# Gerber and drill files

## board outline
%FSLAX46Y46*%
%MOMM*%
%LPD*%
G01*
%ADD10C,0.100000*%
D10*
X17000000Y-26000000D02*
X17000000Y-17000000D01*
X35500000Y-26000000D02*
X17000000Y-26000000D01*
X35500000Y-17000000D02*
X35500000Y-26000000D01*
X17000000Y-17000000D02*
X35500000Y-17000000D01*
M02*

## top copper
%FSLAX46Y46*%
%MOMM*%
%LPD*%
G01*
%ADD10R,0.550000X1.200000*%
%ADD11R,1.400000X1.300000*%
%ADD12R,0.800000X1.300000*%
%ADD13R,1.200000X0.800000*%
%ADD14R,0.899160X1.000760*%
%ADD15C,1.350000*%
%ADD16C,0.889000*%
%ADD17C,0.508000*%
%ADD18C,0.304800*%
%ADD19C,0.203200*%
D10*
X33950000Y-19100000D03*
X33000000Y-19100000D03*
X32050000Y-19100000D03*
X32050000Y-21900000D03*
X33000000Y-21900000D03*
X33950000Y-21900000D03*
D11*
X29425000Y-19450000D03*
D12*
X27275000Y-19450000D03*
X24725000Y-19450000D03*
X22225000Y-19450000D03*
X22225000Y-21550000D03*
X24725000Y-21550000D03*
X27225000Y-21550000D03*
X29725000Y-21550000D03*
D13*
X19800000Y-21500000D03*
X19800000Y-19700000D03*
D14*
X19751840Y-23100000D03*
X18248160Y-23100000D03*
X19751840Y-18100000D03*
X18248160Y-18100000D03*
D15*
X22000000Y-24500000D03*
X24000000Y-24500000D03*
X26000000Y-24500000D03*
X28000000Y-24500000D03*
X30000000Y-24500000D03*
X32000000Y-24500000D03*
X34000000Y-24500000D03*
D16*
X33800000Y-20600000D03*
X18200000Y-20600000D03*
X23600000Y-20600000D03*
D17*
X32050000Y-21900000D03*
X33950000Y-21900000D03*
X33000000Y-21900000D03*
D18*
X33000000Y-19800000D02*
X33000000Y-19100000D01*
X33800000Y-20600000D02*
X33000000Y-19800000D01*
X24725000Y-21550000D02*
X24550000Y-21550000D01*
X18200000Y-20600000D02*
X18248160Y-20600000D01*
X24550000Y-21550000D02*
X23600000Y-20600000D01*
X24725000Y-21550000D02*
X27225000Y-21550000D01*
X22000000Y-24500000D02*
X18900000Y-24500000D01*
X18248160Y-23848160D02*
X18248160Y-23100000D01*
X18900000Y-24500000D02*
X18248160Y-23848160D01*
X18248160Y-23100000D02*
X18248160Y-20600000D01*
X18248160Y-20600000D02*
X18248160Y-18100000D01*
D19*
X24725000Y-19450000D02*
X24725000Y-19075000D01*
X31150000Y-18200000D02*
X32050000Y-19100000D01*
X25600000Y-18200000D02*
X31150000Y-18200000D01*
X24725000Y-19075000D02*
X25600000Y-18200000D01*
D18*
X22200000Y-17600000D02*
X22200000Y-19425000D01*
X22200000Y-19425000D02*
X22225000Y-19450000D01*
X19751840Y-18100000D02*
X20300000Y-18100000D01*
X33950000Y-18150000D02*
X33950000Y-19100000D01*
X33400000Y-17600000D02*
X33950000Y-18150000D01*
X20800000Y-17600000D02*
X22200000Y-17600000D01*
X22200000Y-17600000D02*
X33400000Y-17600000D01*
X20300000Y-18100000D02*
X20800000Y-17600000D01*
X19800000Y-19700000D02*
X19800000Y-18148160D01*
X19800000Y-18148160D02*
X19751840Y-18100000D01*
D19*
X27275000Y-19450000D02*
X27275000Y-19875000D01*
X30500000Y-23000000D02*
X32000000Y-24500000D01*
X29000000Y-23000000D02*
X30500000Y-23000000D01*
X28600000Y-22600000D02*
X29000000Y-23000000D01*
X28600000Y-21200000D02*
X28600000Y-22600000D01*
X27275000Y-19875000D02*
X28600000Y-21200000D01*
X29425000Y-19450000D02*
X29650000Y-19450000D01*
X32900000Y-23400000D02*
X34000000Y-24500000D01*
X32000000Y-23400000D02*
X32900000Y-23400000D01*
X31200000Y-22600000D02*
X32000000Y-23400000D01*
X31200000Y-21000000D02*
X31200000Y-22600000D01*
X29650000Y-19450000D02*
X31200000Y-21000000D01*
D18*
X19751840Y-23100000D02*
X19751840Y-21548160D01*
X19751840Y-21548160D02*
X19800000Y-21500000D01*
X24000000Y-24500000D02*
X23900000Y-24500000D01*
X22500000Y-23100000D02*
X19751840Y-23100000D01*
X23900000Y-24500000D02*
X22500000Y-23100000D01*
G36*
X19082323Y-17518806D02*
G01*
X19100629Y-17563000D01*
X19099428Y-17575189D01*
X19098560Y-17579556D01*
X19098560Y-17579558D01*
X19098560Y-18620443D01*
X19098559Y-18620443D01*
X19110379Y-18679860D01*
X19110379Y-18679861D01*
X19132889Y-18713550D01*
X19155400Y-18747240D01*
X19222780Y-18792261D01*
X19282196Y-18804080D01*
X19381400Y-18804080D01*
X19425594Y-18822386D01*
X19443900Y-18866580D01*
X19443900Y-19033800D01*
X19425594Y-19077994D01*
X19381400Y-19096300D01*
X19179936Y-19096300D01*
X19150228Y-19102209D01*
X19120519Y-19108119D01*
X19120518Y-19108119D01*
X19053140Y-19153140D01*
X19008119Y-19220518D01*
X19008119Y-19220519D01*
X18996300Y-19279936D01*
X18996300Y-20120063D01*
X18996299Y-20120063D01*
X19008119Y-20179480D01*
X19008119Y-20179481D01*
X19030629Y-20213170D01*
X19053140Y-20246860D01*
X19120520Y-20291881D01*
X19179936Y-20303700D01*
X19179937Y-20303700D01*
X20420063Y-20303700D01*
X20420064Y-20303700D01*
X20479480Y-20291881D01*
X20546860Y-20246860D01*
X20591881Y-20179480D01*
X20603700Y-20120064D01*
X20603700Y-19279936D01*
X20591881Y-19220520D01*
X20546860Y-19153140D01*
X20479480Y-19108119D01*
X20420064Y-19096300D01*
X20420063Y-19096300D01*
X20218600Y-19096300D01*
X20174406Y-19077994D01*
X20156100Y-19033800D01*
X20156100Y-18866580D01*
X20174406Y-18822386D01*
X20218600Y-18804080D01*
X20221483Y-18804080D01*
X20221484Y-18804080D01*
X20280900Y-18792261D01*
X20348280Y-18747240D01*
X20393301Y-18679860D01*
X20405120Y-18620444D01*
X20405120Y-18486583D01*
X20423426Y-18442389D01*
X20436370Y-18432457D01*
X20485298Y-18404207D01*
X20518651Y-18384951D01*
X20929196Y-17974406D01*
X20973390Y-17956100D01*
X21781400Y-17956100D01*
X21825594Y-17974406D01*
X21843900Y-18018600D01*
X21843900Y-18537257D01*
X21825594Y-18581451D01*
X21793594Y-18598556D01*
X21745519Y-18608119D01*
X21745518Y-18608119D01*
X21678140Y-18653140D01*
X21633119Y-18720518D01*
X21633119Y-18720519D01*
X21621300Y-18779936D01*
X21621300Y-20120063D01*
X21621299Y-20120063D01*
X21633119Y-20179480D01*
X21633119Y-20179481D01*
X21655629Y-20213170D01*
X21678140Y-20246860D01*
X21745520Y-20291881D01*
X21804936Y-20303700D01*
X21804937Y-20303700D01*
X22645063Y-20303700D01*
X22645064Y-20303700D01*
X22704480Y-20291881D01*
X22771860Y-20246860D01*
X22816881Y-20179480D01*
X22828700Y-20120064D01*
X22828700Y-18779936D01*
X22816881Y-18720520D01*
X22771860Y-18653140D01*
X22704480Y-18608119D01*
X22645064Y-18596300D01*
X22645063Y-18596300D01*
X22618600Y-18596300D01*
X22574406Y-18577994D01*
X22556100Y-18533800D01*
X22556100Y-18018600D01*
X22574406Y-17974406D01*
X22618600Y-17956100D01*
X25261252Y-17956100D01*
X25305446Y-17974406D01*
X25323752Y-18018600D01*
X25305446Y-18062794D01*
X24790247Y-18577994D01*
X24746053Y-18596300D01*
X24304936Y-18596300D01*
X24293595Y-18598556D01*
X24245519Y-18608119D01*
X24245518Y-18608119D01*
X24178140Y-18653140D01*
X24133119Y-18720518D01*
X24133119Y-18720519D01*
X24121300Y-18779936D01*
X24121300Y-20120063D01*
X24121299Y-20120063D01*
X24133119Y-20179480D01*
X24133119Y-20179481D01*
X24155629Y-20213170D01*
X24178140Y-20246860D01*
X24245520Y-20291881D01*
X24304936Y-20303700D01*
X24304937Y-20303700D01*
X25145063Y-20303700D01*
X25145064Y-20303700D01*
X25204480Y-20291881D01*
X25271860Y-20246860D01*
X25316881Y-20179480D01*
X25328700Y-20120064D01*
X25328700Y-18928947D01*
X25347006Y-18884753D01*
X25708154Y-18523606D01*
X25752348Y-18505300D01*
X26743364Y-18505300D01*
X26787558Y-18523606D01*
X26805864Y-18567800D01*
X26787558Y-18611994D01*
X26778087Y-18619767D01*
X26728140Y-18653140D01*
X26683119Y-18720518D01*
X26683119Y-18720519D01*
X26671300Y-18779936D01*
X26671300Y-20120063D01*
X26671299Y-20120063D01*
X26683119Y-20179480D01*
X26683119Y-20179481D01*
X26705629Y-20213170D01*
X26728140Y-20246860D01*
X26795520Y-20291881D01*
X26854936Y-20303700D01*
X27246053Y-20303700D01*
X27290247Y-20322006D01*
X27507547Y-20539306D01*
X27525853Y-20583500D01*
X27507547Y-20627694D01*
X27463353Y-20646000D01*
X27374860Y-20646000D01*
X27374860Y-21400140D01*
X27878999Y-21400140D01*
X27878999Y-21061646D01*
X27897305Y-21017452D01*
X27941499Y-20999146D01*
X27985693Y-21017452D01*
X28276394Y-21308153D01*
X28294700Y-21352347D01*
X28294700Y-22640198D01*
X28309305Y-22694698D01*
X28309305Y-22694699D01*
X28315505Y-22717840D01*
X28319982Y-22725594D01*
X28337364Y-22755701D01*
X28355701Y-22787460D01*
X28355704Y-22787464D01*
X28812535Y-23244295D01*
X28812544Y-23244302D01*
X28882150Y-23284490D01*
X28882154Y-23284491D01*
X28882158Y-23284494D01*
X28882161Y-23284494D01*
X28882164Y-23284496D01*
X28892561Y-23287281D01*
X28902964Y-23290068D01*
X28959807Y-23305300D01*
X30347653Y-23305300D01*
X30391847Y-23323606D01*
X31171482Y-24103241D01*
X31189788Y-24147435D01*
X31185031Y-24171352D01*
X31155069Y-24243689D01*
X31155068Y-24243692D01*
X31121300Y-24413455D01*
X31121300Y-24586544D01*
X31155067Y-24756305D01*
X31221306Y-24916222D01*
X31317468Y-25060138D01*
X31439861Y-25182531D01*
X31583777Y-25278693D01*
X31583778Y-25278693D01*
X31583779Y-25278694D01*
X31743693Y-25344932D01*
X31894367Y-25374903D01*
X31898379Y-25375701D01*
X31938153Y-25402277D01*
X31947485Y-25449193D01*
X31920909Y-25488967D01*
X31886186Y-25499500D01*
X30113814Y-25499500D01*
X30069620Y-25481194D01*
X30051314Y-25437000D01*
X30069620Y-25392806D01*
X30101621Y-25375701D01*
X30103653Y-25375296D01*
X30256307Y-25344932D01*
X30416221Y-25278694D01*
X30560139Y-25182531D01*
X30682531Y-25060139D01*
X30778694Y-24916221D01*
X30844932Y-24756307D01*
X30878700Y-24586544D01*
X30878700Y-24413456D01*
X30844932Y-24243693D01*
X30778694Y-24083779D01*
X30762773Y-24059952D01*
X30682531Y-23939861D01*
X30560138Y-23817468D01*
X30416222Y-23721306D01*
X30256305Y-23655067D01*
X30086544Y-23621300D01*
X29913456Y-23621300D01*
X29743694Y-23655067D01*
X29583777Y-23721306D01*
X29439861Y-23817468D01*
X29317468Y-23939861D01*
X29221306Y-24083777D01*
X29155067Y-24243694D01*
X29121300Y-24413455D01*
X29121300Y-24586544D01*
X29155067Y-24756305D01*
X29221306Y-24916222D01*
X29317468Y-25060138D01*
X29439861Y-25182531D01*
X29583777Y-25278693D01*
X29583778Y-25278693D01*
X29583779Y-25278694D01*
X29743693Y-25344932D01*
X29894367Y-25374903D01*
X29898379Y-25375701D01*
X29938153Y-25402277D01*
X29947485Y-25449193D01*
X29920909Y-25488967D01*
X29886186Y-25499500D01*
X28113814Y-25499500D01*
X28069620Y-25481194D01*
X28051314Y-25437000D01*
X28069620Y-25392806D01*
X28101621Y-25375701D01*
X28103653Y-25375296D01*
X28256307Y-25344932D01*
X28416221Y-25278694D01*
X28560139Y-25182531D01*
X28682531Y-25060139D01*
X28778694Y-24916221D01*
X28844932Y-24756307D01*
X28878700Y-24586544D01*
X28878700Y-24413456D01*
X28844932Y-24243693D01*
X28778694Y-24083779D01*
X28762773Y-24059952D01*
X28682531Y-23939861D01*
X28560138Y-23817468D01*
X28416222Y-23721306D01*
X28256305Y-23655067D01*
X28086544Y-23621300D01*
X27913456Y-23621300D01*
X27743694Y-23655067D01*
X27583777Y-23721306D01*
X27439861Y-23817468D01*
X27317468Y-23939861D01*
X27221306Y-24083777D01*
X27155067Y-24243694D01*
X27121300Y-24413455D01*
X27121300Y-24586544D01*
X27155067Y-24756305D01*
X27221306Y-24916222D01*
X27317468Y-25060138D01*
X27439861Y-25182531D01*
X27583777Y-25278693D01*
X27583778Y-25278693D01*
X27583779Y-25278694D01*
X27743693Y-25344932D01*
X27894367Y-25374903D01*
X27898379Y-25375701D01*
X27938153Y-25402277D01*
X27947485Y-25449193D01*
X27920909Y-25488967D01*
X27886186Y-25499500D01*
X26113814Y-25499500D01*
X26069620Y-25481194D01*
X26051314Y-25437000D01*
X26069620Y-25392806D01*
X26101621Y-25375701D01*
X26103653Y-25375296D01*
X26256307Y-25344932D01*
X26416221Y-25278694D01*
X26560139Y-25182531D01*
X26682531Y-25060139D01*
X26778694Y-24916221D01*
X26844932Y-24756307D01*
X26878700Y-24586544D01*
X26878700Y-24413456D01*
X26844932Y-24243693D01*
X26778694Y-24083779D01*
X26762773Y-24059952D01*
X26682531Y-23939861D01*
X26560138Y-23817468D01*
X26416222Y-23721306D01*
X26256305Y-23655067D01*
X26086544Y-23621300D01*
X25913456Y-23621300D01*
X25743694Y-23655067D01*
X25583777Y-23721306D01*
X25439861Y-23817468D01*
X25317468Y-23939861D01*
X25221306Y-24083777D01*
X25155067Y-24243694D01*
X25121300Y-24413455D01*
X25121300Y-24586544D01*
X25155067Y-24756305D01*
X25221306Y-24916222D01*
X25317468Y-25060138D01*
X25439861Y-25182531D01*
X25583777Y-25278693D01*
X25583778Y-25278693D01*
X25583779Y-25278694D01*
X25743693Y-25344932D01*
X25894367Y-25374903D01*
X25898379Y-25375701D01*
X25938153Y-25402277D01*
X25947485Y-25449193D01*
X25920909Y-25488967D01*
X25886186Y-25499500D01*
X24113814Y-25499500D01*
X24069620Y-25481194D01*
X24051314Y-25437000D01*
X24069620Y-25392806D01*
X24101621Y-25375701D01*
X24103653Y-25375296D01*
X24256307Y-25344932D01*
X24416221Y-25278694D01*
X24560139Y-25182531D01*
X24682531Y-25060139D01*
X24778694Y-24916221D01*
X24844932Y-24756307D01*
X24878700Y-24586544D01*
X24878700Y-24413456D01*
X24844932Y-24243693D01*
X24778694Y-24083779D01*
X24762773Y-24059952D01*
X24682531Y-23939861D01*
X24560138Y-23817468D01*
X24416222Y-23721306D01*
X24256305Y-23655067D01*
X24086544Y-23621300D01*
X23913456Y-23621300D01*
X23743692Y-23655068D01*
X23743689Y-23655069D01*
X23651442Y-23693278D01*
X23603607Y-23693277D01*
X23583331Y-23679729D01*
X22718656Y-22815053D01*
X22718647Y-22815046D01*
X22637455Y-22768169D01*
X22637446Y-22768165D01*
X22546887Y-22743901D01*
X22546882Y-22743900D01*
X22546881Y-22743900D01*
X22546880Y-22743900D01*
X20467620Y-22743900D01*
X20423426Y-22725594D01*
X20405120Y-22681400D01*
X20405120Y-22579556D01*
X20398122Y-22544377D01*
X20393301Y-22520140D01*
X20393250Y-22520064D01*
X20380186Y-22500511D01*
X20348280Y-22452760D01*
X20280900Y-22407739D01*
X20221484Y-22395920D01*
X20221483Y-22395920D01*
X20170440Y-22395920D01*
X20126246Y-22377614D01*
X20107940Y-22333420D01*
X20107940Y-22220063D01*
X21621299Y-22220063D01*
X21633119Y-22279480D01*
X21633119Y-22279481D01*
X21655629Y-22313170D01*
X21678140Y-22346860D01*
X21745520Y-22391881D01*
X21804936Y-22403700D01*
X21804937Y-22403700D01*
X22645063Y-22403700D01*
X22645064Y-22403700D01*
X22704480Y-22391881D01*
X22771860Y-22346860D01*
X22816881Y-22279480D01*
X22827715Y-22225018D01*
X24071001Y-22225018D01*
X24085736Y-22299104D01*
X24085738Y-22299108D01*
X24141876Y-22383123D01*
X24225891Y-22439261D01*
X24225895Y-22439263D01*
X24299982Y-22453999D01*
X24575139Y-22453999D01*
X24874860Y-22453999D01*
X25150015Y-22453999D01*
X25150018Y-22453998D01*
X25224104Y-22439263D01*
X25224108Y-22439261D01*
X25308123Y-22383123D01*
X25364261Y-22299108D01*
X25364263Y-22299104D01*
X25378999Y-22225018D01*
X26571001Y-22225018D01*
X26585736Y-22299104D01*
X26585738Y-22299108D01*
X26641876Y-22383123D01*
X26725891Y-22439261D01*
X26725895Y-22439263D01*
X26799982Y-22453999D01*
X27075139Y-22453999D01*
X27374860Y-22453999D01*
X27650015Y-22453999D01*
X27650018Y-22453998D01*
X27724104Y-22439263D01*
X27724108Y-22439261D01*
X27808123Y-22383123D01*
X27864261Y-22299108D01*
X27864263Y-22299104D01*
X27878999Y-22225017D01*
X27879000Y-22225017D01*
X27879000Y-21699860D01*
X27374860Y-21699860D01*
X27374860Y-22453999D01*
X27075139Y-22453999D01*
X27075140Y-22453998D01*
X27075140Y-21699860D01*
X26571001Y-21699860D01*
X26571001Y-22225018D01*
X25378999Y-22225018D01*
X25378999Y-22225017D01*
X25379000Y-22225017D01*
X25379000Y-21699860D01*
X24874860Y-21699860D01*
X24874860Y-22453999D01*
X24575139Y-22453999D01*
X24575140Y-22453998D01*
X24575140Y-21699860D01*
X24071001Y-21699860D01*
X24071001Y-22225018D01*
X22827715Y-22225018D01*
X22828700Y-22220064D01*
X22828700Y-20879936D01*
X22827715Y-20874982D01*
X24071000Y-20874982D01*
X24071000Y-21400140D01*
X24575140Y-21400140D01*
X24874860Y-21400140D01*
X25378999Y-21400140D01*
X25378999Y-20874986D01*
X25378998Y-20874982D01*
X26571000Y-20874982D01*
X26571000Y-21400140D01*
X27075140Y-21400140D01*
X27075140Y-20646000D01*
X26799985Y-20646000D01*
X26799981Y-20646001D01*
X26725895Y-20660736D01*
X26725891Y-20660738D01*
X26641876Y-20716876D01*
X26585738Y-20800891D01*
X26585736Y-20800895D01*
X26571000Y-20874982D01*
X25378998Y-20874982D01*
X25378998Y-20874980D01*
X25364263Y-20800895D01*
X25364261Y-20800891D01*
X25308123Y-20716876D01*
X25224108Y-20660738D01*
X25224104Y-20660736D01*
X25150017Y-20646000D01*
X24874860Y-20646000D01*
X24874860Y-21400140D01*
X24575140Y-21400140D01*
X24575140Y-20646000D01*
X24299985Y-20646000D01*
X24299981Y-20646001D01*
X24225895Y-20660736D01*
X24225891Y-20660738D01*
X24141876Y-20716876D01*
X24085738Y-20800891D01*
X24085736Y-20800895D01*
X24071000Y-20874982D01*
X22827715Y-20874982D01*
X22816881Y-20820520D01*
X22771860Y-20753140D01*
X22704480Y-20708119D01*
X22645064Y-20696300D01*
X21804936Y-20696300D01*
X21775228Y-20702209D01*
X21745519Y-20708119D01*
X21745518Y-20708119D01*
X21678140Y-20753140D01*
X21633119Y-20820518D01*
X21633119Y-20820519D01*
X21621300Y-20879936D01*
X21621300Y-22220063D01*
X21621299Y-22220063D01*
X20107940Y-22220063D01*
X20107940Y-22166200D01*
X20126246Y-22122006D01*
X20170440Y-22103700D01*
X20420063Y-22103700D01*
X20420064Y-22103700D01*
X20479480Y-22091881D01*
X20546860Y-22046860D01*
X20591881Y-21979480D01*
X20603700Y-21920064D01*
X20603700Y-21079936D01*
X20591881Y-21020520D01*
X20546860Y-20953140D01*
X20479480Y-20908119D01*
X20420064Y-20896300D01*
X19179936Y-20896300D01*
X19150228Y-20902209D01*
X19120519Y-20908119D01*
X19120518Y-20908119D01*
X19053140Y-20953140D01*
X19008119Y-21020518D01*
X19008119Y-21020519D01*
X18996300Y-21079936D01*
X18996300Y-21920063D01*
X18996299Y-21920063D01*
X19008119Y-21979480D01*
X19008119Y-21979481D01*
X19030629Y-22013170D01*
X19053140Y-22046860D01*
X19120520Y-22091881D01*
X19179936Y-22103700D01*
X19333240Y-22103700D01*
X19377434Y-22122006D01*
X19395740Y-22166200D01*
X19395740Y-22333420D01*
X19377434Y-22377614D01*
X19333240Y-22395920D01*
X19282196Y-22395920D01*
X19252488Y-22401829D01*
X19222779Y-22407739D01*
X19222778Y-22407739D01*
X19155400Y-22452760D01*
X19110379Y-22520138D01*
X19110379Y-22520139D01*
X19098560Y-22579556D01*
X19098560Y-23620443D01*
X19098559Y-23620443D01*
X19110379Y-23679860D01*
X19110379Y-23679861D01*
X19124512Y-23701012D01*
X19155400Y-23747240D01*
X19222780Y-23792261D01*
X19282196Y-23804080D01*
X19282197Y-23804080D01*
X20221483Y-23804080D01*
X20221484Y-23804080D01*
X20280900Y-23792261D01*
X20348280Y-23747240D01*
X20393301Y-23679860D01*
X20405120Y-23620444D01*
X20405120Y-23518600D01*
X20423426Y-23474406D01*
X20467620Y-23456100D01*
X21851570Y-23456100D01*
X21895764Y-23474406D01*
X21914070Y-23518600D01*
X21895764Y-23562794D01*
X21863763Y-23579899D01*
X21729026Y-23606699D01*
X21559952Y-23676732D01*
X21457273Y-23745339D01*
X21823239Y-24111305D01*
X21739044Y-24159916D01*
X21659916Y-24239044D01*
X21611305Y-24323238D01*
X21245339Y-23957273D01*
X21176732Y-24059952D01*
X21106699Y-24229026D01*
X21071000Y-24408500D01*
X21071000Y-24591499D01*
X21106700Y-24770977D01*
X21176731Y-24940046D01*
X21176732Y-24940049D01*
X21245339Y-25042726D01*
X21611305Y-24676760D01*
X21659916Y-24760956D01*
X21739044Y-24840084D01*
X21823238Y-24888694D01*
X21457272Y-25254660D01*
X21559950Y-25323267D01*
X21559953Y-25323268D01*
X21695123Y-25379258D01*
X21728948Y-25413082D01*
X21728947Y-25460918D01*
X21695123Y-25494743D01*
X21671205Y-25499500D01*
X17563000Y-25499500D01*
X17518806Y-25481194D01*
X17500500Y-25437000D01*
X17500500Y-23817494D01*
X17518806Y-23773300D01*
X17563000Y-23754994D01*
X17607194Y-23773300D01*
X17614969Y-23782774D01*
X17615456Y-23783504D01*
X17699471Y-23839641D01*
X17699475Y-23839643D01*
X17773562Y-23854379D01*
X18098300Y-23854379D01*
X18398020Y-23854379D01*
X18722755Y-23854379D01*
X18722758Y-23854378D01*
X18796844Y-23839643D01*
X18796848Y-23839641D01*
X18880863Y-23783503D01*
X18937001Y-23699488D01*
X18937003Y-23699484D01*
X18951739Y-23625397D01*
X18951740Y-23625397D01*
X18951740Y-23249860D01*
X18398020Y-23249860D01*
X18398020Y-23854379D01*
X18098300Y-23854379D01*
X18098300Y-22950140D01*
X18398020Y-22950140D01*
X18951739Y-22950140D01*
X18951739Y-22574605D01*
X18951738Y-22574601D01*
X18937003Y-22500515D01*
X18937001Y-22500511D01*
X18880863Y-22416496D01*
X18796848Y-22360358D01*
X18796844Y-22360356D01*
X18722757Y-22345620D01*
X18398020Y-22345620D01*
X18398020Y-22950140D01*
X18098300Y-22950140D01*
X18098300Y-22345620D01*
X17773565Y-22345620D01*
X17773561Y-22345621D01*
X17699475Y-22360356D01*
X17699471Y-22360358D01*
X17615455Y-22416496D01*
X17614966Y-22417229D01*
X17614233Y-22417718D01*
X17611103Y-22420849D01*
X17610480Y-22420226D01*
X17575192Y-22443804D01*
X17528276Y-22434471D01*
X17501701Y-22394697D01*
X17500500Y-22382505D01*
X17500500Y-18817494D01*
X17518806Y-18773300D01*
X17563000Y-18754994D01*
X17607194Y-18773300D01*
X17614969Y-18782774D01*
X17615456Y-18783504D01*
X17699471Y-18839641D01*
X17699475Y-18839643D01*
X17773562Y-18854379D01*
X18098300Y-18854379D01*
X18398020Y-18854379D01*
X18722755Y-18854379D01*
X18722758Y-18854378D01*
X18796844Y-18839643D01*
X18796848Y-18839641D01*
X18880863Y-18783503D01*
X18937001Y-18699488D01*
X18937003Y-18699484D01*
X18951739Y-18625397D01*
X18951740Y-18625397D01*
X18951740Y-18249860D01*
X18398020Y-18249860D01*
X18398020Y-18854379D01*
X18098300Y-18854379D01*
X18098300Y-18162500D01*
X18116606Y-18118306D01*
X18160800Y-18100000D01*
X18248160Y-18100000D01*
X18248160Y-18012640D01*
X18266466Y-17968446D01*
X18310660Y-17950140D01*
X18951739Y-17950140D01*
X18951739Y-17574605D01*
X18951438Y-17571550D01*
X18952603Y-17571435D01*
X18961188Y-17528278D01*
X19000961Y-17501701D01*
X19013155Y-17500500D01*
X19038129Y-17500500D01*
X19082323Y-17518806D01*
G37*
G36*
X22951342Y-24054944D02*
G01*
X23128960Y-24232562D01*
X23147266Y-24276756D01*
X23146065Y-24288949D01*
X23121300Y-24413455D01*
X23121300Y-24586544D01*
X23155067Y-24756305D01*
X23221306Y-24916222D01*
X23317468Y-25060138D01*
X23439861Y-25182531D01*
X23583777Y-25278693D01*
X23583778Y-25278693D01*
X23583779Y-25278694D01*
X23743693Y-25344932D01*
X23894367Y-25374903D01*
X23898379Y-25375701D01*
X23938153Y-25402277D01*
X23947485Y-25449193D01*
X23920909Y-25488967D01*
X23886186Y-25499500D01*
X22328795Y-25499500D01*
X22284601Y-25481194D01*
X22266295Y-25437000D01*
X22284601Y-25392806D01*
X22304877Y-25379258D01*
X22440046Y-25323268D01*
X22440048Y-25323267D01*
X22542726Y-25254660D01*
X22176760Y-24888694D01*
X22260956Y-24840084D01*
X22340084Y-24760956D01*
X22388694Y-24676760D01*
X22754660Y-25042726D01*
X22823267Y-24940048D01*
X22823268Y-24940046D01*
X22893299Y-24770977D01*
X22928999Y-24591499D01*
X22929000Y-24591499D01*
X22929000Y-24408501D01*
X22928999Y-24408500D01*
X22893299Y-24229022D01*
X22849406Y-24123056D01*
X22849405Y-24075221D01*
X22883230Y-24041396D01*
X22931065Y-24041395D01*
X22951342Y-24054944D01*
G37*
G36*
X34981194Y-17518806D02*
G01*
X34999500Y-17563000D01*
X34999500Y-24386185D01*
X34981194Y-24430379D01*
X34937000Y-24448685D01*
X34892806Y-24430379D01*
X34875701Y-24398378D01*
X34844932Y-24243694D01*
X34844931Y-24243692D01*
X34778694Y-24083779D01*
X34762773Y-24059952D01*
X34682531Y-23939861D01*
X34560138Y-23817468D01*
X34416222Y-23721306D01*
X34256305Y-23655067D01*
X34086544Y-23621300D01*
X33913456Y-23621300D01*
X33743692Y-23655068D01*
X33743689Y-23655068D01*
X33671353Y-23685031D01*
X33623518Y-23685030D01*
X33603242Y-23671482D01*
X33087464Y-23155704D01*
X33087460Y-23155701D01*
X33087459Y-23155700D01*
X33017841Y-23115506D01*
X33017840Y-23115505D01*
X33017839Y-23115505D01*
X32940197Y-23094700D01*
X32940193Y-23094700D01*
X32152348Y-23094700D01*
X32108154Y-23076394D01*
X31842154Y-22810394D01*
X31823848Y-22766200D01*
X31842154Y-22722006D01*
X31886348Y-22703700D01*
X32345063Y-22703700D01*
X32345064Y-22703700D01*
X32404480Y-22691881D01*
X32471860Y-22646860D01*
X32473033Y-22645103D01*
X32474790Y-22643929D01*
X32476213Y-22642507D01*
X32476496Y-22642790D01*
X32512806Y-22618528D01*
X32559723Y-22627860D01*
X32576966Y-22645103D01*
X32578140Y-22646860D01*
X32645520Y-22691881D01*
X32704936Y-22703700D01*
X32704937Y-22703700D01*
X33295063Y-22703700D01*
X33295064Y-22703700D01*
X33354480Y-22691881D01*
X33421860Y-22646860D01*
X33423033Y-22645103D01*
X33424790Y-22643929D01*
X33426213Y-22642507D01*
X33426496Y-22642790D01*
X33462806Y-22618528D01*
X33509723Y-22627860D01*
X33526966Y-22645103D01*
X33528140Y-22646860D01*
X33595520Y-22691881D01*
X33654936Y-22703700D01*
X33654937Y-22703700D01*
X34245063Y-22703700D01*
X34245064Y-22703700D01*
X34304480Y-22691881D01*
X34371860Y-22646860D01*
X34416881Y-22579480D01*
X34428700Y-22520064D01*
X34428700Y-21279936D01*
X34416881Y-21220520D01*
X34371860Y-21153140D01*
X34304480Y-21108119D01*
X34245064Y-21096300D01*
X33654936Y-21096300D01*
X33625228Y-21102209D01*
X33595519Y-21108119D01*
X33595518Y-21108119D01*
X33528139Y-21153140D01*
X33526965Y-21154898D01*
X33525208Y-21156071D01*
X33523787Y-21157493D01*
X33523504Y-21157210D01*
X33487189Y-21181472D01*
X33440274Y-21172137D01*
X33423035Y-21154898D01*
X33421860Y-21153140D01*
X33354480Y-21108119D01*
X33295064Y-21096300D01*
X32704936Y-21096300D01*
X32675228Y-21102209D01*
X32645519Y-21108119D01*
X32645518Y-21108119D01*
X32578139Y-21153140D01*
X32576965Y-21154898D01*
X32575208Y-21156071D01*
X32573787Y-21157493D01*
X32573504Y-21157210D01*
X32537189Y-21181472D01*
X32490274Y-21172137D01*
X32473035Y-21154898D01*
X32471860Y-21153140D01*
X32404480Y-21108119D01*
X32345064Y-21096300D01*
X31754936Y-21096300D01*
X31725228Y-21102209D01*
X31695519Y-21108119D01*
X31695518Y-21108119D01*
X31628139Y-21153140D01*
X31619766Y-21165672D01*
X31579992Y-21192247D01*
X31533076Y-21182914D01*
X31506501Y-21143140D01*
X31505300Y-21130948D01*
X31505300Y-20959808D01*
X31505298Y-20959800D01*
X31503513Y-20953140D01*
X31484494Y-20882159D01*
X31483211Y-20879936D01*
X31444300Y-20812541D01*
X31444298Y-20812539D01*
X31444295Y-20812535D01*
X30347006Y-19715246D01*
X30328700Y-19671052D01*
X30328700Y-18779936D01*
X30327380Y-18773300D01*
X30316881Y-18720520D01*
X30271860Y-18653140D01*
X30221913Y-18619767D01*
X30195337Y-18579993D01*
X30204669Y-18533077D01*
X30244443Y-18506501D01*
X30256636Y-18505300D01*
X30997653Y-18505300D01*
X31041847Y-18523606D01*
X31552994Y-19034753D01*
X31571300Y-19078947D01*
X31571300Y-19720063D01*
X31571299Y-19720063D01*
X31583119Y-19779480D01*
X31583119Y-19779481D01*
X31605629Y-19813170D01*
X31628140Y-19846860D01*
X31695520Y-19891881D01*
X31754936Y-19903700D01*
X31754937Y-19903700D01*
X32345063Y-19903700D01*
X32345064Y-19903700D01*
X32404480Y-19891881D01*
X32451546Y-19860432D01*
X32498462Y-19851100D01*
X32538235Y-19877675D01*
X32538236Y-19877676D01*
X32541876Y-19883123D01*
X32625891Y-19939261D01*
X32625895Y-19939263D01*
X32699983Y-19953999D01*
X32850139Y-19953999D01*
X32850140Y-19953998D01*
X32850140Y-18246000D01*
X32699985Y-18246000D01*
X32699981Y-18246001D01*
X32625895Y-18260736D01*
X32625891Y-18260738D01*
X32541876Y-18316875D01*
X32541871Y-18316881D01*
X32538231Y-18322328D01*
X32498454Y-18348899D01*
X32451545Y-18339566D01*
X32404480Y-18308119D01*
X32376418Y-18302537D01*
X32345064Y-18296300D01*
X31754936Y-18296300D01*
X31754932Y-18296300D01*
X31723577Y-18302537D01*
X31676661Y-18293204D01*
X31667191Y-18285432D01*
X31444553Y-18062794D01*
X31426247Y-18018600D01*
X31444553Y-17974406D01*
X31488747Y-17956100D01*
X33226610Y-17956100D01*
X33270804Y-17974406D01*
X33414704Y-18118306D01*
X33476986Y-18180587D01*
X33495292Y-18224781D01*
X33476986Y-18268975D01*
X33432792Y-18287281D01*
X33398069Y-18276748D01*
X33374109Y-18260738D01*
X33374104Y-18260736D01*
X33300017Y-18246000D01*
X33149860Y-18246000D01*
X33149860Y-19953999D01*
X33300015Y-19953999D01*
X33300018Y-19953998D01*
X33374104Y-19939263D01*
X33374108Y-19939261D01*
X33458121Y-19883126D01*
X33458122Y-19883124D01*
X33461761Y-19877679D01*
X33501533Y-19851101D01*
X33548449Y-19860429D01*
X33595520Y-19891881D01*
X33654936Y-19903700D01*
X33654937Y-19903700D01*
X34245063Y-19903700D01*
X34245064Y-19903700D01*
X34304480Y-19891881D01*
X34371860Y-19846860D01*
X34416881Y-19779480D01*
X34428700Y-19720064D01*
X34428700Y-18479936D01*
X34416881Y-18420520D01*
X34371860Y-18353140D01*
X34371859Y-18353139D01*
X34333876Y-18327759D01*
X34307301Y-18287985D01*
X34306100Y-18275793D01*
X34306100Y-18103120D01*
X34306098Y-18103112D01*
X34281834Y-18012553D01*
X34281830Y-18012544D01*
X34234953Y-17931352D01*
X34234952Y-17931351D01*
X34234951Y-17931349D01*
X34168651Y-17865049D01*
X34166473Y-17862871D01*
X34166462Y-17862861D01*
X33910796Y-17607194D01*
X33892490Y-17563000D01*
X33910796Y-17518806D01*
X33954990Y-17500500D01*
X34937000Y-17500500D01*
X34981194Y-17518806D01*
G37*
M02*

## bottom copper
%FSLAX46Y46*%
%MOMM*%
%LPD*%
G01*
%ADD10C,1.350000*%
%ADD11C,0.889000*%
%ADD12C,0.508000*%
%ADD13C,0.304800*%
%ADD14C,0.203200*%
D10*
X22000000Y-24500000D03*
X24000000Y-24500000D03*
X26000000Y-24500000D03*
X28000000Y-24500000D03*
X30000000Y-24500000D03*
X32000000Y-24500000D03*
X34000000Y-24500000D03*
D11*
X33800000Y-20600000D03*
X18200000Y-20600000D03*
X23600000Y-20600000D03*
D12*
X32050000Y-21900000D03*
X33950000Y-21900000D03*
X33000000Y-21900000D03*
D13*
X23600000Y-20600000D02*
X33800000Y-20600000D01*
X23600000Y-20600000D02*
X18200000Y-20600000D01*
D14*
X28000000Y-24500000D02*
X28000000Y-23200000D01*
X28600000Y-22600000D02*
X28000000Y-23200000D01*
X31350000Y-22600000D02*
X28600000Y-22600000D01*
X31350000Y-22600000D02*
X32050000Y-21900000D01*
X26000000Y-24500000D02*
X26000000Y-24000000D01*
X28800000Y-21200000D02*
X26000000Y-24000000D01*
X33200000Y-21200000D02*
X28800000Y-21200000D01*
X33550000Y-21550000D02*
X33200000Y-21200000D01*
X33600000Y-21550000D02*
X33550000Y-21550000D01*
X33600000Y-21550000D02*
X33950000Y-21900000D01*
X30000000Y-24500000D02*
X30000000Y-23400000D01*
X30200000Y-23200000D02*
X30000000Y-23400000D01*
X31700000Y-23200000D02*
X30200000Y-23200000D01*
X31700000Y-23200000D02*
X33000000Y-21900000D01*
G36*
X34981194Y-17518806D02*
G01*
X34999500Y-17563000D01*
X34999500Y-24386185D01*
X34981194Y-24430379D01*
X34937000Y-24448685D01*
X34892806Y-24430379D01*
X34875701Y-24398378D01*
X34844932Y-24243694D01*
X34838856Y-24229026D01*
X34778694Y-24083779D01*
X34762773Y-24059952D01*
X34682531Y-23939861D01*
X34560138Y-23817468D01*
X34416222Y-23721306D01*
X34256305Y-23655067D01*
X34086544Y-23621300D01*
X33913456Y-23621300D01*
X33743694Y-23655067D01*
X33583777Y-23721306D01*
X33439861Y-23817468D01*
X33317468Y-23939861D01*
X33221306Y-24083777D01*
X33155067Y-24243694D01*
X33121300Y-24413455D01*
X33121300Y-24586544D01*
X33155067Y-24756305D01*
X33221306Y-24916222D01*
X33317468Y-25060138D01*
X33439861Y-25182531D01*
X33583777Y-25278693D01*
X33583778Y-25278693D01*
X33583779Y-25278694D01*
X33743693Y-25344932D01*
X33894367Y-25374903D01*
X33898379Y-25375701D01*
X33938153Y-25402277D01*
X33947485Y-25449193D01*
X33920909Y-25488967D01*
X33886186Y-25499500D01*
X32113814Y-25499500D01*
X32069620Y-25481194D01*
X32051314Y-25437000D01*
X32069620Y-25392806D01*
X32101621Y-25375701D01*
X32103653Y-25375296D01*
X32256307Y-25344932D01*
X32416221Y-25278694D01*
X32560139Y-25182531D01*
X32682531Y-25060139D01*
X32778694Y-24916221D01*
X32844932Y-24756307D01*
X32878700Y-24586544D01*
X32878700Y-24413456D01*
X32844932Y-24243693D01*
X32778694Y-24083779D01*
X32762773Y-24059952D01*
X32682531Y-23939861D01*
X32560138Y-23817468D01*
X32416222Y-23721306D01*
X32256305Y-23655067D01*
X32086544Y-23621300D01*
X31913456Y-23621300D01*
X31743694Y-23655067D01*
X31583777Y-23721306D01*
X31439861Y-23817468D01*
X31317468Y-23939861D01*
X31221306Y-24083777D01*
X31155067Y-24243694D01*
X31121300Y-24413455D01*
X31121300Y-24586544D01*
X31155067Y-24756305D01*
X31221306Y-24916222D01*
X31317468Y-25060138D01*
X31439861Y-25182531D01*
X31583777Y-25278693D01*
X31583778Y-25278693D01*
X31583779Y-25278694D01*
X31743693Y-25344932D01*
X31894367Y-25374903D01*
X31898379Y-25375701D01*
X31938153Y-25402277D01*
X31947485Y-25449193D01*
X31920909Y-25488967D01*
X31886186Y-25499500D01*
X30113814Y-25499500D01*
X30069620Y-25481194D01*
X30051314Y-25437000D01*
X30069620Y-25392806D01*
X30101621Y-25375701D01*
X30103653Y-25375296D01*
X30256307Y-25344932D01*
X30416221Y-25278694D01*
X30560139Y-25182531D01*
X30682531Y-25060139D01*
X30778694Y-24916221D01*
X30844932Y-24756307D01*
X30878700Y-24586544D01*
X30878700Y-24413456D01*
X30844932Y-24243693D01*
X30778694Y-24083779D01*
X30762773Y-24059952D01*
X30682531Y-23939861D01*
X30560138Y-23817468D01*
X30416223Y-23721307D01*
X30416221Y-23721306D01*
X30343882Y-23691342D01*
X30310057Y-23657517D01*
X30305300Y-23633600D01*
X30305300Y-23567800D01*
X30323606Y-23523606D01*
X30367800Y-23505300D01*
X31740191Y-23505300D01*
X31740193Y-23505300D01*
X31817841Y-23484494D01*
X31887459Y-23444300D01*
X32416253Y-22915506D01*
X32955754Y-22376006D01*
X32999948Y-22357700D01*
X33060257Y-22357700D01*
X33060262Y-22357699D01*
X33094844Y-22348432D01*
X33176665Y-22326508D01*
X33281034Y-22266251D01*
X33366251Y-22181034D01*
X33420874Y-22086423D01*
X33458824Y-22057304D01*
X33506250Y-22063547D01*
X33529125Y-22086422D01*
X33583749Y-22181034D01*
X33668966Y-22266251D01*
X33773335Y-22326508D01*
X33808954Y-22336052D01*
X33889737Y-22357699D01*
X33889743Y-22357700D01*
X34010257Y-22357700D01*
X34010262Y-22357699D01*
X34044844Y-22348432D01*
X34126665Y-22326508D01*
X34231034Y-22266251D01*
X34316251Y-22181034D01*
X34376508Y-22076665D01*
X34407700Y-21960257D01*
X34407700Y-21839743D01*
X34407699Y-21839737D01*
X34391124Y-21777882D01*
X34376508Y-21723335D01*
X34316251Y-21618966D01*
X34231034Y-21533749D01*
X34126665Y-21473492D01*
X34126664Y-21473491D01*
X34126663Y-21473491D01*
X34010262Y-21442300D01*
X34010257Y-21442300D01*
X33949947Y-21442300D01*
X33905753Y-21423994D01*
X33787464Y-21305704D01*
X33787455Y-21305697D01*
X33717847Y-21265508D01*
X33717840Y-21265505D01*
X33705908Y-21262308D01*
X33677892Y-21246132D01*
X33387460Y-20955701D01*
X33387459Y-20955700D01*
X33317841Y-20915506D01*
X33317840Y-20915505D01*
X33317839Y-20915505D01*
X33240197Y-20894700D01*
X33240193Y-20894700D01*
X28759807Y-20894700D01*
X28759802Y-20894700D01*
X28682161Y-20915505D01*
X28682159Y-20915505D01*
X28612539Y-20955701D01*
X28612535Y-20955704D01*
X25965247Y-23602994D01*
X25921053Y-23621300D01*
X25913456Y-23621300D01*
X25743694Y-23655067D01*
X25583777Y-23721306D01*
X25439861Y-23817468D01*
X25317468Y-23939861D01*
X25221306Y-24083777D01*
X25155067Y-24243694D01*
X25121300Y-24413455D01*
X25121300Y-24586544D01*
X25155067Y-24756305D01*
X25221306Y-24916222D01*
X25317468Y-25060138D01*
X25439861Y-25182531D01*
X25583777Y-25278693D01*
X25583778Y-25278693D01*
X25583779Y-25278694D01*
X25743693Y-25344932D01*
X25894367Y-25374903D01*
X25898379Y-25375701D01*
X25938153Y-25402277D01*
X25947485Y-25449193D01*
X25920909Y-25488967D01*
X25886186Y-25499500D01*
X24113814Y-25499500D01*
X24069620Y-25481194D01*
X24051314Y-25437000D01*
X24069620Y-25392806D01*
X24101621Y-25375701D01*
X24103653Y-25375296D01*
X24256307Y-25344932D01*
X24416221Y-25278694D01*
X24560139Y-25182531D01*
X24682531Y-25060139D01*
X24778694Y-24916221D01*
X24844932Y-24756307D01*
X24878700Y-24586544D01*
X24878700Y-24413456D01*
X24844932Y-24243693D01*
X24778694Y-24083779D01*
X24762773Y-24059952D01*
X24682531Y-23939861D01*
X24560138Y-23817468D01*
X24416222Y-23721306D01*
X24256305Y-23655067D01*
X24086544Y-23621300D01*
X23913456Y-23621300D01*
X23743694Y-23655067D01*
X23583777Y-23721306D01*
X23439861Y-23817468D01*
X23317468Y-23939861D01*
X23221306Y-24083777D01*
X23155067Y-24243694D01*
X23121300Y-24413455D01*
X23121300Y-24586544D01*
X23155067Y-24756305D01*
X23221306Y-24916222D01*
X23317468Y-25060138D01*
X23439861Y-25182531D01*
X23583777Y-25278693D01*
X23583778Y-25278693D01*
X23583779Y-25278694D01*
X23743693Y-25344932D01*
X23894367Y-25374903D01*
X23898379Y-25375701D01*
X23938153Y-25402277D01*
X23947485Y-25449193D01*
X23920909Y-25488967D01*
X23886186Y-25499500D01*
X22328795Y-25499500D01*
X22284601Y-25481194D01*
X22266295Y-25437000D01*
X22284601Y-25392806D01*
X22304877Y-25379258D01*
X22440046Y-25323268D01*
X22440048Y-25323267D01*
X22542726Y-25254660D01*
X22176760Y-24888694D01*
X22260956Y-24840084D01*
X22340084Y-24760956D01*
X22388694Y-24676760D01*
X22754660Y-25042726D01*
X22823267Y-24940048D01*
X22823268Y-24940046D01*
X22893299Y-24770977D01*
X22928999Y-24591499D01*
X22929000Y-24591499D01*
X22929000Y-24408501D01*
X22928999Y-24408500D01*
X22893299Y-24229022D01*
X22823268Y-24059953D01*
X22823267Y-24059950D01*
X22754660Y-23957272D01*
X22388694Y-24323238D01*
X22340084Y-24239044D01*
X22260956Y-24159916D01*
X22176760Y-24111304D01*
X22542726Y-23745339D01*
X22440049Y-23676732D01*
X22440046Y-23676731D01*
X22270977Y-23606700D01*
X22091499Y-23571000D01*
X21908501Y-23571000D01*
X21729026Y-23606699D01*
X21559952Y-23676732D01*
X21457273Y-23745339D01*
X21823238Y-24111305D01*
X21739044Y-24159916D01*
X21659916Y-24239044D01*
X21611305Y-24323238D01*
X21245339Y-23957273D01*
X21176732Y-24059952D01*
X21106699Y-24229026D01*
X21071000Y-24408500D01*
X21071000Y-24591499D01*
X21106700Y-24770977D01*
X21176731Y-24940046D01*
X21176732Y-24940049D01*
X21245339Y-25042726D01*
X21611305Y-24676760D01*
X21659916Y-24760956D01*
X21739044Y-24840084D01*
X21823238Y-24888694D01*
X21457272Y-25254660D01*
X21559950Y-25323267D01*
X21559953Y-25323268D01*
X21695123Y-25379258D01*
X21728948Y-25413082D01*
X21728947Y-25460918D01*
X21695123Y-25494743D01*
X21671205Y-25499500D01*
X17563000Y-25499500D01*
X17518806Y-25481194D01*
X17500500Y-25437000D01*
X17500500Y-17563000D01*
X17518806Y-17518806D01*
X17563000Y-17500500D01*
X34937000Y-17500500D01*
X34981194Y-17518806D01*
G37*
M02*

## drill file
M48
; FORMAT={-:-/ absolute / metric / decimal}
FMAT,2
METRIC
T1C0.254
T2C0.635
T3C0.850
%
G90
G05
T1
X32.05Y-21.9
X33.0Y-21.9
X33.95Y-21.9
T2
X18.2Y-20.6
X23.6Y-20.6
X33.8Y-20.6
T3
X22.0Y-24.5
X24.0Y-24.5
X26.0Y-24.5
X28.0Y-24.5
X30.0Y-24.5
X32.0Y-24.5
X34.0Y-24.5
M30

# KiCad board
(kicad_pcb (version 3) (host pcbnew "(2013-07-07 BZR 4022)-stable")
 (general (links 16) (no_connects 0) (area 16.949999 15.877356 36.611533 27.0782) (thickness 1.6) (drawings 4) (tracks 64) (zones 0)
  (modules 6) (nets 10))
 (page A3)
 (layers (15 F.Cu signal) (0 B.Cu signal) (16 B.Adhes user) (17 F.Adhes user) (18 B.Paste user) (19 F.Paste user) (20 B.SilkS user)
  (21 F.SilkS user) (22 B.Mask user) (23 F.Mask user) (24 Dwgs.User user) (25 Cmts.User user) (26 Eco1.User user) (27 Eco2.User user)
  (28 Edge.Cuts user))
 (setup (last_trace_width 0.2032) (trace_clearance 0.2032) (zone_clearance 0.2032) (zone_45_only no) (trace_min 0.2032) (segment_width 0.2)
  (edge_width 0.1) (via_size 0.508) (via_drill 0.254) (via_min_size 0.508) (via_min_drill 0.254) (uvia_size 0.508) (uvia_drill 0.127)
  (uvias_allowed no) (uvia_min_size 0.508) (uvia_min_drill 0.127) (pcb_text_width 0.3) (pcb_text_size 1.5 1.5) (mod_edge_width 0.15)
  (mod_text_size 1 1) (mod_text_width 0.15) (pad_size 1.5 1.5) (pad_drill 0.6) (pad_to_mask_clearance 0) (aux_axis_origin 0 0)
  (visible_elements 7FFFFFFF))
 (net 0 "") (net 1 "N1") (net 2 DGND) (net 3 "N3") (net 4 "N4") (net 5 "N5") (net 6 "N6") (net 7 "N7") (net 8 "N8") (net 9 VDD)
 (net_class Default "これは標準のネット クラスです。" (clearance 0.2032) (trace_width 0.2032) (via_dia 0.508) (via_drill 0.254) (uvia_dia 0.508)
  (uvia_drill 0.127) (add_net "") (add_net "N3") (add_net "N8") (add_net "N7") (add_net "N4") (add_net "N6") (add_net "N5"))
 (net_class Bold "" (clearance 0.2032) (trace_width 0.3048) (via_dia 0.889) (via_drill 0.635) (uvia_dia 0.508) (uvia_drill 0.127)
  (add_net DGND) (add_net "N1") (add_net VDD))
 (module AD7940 (layer F.Cu) (at 33 20.5 180)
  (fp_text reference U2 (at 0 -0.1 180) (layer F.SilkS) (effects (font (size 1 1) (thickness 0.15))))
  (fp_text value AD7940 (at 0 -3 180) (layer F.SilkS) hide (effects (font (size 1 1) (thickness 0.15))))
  (pad 1 smd rect (at -0.95 1.4 180) (size 0.55 1.2) (layers F.Cu F.Paste F.Mask) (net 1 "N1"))
  (pad 2 smd rect (at 0 1.4 180) (size 0.55 1.2) (layers F.Cu F.Paste F.Mask) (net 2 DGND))
  (pad 3 smd rect (at 0.95 1.4 180) (size 0.55 1.2) (layers F.Cu F.Paste F.Mask) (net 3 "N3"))
  (pad 4 smd rect (at 0.95 -1.4 180) (size 0.55 1.2) (layers F.Cu F.Paste F.Mask) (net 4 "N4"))
  (pad 5 smd rect (at 0 -1.4 180) (size 0.55 1.2) (layers F.Cu F.Paste F.Mask) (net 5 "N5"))
  (pad 6 smd rect (at -0.95 -1.4 180) (size 0.55 1.2) (layers F.Cu F.Paste F.Mask) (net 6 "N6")))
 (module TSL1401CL (layer F.Cu) (at 26 20.5 180)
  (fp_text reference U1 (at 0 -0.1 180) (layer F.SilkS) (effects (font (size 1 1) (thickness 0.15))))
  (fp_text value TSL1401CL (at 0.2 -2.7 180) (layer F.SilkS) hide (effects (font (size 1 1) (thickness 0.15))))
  (pad 1 smd rect (at -3.425 1.05 180) (size 1.4 1.3) (layers F.Cu F.Paste F.Mask) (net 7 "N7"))
  (pad 2 smd rect (at -1.275 1.05 180) (size 0.8 1.3) (layers F.Cu F.Paste F.Mask) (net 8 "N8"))
  (pad 3 smd rect (at 1.275 1.05 180) (size 0.8 1.3) (layers F.Cu F.Paste F.Mask) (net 3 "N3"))
  (pad 4 smd rect (at 3.775 1.05 180) (size 0.8 1.3) (layers F.Cu F.Paste F.Mask) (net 1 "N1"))
  (pad 5 smd rect (at 3.775 -1.05 180) (size 0.8 1.3) (layers F.Cu F.Paste F.Mask))
  (pad 6 smd rect (at 1.275 -1.05 180) (size 0.8 1.3) (layers F.Cu F.Paste F.Mask) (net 2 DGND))
  (pad 7 smd rect (at -1.225 -1.05 180) (size 0.8 1.3) (layers F.Cu F.Paste F.Mask) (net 2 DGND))
  (pad 8 smd rect (at -3.725 -1.05 180) (size 0.8 1.3) (layers F.Cu F.Paste F.Mask)))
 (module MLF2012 (layer F.Cu) (at 19.8 20.6 90)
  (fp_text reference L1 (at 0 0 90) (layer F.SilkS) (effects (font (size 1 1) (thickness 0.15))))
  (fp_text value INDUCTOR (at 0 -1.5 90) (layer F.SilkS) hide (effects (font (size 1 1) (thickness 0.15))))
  (pad 1 smd rect (at -0.9 0 90) (size 0.8 1.2) (layers F.Cu F.Paste F.Mask) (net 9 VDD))
  (pad 2 smd rect (at 0.9 0 90) (size 0.8 1.2) (layers F.Cu F.Paste F.Mask) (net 1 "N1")))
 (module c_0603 (layer F.Cu) (at 19 23.1)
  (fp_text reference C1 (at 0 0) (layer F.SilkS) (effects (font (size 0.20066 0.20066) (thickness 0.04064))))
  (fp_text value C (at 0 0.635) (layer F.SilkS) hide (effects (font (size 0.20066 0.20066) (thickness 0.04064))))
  (pad 1 smd rect (at 0.75184 0) (size 0.89916 1.00076) (layers F.Cu F.Paste F.Mask) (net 9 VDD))
  (pad 2 smd rect (at -0.75184 0) (size 0.89916 1.00076) (layers F.Cu F.Paste F.Mask) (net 2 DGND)))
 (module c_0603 (layer F.Cu) (at 19 18.1)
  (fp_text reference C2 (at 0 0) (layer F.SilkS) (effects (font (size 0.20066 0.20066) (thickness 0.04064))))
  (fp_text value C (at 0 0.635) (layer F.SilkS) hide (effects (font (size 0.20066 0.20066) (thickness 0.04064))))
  (pad 1 smd rect (at 0.75184 0) (size 0.89916 1.00076) (layers F.Cu F.Paste F.Mask) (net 1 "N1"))
  (pad 2 smd rect (at -0.75184 0) (size 0.89916 1.00076) (layers F.Cu F.Paste F.Mask) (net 2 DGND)))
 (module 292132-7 (layer F.Cu) (at 28 24.5)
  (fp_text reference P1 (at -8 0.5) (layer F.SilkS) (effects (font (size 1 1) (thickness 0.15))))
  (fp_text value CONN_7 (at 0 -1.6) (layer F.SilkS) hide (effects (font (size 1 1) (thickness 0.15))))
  (pad 1 thru_hole circle (at -6 0) (size 1.35 1.35) (drill 0.85) (layers *.Cu *.Mask F.SilkS) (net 2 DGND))
  (pad 2 thru_hole circle (at -4 0) (size 1.35 1.35) (drill 0.85) (layers *.Cu *.Mask F.SilkS) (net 9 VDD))
  (pad 3 thru_hole circle (at -2 0) (size 1.35 1.35) (drill 0.85) (layers *.Cu *.Mask F.SilkS) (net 6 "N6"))
  (pad 4 thru_hole circle (at 0 0) (size 1.35 1.35) (drill 0.85) (layers *.Cu *.Mask F.SilkS) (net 4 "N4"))
  (pad 5 thru_hole circle (at 2 0) (size 1.35 1.35) (drill 0.85) (layers *.Cu *.Mask F.SilkS) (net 5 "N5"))
  (pad 6 thru_hole circle (at 4 0) (size 1.35 1.35) (drill 0.85) (layers *.Cu *.Mask F.SilkS) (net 8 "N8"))
  (pad 7 thru_hole circle (at 6 0) (size 1.35 1.35) (drill 0.85) (layers *.Cu *.Mask F.SilkS) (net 7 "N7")))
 (gr_line (start 17 26) (end 17 17) (angle 90) (layer Edge.Cuts) (width 0.1))
 (gr_line (start 35.5 26) (end 17 26) (angle 90) (layer Edge.Cuts) (width 0.1))
 (gr_line (start 35.5 17) (end 35.5 26) (angle 90) (layer Edge.Cuts) (width 0.1))
 (gr_line (start 17 17) (end 35.5 17) (angle 90) (layer Edge.Cuts) (width 0.1))
 (segment (start 23.6 20.6) (end 33.8 20.6) (width 0.3048) (layer B.Cu) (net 2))
 (segment (start 33 19.8) (end 33 19.1) (width 0.3048) (layer F.Cu) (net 2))
 (segment (start 33.8 20.6) (end 33 19.8) (width 0.3048) (layer F.Cu) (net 2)) (via (at 33.8 20.6) (size 0.889) (layers F.Cu B.Cu) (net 2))
 (segment (start 24.725 21.55) (end 24.55 21.55) (width 0.3048) (layer F.Cu) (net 2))
 (segment (start 18.2 20.6) (end 18.24816 20.6) (width 0.3048) (layer F.Cu) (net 2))
 (via (at 18.2 20.6) (size 0.889) (layers F.Cu B.Cu) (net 2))
 (segment (start 23.6 20.6) (end 18.2 20.6) (width 0.3048) (layer B.Cu) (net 2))
 (via (at 23.6 20.6) (size 0.889) (layers F.Cu B.Cu) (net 2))
 (segment (start 24.55 21.55) (end 23.6 20.6) (width 0.3048) (layer F.Cu) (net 2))
 (segment (start 24.725 21.55) (end 27.225 21.55) (width 0.3048) (layer F.Cu) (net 2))
 (segment (start 22 24.5) (end 18.9 24.5) (width 0.3048) (layer F.Cu) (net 2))
 (segment (start 18.24816 23.84816) (end 18.24816 23.1) (width 0.3048) (layer F.Cu) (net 2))
 (segment (start 18.9 24.5) (end 18.24816 23.84816) (width 0.3048) (layer F.Cu) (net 2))
 (segment (start 18.24816 23.1) (end 18.24816 20.6) (width 0.3048) (layer F.Cu) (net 2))
 (segment (start 18.24816 20.6) (end 18.24816 18.1) (width 0.3048) (layer F.Cu) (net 2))
 (segment (start 24.725 19.45) (end 24.725 19.075) (width 0.2032) (layer F.Cu) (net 3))
 (segment (start 31.15 18.2) (end 32.05 19.1) (width 0.2032) (layer F.Cu) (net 3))
 (segment (start 25.6 18.2) (end 31.15 18.2) (width 0.2032) (layer F.Cu) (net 3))
 (segment (start 24.725 19.075) (end 25.6 18.2) (width 0.2032) (layer F.Cu) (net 3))
 (segment (start 22.2 17.6) (end 22.2 19.425) (width 0.3048) (layer F.Cu) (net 1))
 (segment (start 22.2 19.425) (end 22.225 19.45) (width 0.3048) (layer F.Cu) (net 1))
 (segment (start 19.75184 18.1) (end 20.3 18.1) (width 0.3048) (layer F.Cu) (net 1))
 (segment (start 33.95 18.15) (end 33.95 19.1) (width 0.3048) (layer F.Cu) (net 1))
 (segment (start 33.4 17.6) (end 33.95 18.15) (width 0.3048) (layer F.Cu) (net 1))
 (segment (start 20.8 17.6) (end 22.2 17.6) (width 0.3048) (layer F.Cu) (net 1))
 (segment (start 22.2 17.6) (end 33.4 17.6) (width 0.3048) (layer F.Cu) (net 1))
 (segment (start 20.3 18.1) (end 20.8 17.6) (width 0.3048) (layer F.Cu) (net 1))
 (segment (start 19.8 19.7) (end 19.8 18.14816) (width 0.3048) (layer F.Cu) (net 1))
 (segment (start 19.8 18.14816) (end 19.75184 18.1) (width 0.3048) (layer F.Cu) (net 1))
 (segment (start 27.275 19.45) (end 27.275 19.875) (width 0.2032) (layer F.Cu) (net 8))
 (segment (start 30.5 23) (end 32 24.5) (width 0.2032) (layer F.Cu) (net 8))
 (segment (start 29 23) (end 30.5 23) (width 0.2032) (layer F.Cu) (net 8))
 (segment (start 28.6 22.6) (end 29 23) (width 0.2032) (layer F.Cu) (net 8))
 (segment (start 28.6 21.2) (end 28.6 22.6) (width 0.2032) (layer F.Cu) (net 8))
 (segment (start 27.275 19.875) (end 28.6 21.2) (width 0.2032) (layer F.Cu) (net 8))
 (segment (start 29.425 19.45) (end 29.65 19.45) (width 0.2032) (layer F.Cu) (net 7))
 (segment (start 32.9 23.4) (end 34 24.5) (width 0.2032) (layer F.Cu) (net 7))
 (segment (start 32 23.4) (end 32.9 23.4) (width 0.2032) (layer F.Cu) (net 7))
 (segment (start 31.2 22.6) (end 32 23.4) (width 0.2032) (layer F.Cu) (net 7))
 (segment (start 31.2 21) (end 31.2 22.6) (width 0.2032) (layer F.Cu) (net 7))
 (segment (start 29.65 19.45) (end 31.2 21) (width 0.2032) (layer F.Cu) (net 7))
 (via (at 32.05 21.9) (size 0.508) (layers F.Cu B.Cu) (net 4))
 (segment (start 28 24.5) (end 28 23.2) (width 0.2032) (layer B.Cu) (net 4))
 (segment (start 28.6 22.6) (end 28 23.2) (width 0.2032) (layer B.Cu) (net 4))
 (segment (start 31.35 22.6) (end 28.6 22.6) (width 0.2032) (layer B.Cu) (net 4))
 (segment (start 31.35 22.6) (end 32.05 21.9) (width 0.2032) (layer B.Cu) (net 4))
 (via (at 33.95 21.9) (size 0.508) (layers F.Cu B.Cu) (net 6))
 (segment (start 26 24.5) (end 26 24) (width 0.2032) (layer B.Cu) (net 6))
 (segment (start 28.8 21.2) (end 26 24) (width 0.2032) (layer B.Cu) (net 6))
 (segment (start 33.2 21.2) (end 28.8 21.2) (width 0.2032) (layer B.Cu) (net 6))
 (segment (start 33.55 21.55) (end 33.2 21.2) (width 0.2032) (layer B.Cu) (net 6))
 (segment (start 33.6 21.55) (end 33.55 21.55) (width 0.2032) (layer B.Cu) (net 6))
 (segment (start 33.6 21.55) (end 33.95 21.9) (width 0.2032) (layer B.Cu) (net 6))
 (via (at 33 21.9) (size 0.508) (layers F.Cu B.Cu) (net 5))
 (segment (start 30 24.5) (end 30 23.4) (width 0.2032) (layer B.Cu) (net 5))
 (segment (start 30.2 23.2) (end 30 23.4) (width 0.2032) (layer B.Cu) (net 5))
 (segment (start 31.7 23.2) (end 30.2 23.2) (width 0.2032) (layer B.Cu) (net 5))
 (segment (start 31.7 23.2) (end 33 21.9) (width 0.2032) (layer B.Cu) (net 5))
 (segment (start 19.75184 23.1) (end 19.75184 21.54816) (width 0.3048) (layer F.Cu) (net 9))
 (segment (start 19.75184 21.54816) (end 19.8 21.5) (width 0.3048) (layer F.Cu) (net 9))
 (segment (start 24 24.5) (end 23.9 24.5) (width 0.3048) (layer F.Cu) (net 9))
 (segment (start 22.5 23.1) (end 19.75184 23.1) (width 0.3048) (layer F.Cu) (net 9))
 (segment (start 23.9 24.5) (end 22.5 23.1) (width 0.3048) (layer F.Cu) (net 9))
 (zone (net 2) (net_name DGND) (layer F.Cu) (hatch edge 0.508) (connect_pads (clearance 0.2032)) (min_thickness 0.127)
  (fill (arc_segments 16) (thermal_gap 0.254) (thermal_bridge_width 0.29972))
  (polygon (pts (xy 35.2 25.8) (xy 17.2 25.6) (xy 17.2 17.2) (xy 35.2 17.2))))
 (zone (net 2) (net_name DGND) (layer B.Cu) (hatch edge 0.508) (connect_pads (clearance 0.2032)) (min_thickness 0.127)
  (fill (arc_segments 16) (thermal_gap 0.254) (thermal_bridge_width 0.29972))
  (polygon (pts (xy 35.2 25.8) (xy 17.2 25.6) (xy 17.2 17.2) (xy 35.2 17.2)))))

